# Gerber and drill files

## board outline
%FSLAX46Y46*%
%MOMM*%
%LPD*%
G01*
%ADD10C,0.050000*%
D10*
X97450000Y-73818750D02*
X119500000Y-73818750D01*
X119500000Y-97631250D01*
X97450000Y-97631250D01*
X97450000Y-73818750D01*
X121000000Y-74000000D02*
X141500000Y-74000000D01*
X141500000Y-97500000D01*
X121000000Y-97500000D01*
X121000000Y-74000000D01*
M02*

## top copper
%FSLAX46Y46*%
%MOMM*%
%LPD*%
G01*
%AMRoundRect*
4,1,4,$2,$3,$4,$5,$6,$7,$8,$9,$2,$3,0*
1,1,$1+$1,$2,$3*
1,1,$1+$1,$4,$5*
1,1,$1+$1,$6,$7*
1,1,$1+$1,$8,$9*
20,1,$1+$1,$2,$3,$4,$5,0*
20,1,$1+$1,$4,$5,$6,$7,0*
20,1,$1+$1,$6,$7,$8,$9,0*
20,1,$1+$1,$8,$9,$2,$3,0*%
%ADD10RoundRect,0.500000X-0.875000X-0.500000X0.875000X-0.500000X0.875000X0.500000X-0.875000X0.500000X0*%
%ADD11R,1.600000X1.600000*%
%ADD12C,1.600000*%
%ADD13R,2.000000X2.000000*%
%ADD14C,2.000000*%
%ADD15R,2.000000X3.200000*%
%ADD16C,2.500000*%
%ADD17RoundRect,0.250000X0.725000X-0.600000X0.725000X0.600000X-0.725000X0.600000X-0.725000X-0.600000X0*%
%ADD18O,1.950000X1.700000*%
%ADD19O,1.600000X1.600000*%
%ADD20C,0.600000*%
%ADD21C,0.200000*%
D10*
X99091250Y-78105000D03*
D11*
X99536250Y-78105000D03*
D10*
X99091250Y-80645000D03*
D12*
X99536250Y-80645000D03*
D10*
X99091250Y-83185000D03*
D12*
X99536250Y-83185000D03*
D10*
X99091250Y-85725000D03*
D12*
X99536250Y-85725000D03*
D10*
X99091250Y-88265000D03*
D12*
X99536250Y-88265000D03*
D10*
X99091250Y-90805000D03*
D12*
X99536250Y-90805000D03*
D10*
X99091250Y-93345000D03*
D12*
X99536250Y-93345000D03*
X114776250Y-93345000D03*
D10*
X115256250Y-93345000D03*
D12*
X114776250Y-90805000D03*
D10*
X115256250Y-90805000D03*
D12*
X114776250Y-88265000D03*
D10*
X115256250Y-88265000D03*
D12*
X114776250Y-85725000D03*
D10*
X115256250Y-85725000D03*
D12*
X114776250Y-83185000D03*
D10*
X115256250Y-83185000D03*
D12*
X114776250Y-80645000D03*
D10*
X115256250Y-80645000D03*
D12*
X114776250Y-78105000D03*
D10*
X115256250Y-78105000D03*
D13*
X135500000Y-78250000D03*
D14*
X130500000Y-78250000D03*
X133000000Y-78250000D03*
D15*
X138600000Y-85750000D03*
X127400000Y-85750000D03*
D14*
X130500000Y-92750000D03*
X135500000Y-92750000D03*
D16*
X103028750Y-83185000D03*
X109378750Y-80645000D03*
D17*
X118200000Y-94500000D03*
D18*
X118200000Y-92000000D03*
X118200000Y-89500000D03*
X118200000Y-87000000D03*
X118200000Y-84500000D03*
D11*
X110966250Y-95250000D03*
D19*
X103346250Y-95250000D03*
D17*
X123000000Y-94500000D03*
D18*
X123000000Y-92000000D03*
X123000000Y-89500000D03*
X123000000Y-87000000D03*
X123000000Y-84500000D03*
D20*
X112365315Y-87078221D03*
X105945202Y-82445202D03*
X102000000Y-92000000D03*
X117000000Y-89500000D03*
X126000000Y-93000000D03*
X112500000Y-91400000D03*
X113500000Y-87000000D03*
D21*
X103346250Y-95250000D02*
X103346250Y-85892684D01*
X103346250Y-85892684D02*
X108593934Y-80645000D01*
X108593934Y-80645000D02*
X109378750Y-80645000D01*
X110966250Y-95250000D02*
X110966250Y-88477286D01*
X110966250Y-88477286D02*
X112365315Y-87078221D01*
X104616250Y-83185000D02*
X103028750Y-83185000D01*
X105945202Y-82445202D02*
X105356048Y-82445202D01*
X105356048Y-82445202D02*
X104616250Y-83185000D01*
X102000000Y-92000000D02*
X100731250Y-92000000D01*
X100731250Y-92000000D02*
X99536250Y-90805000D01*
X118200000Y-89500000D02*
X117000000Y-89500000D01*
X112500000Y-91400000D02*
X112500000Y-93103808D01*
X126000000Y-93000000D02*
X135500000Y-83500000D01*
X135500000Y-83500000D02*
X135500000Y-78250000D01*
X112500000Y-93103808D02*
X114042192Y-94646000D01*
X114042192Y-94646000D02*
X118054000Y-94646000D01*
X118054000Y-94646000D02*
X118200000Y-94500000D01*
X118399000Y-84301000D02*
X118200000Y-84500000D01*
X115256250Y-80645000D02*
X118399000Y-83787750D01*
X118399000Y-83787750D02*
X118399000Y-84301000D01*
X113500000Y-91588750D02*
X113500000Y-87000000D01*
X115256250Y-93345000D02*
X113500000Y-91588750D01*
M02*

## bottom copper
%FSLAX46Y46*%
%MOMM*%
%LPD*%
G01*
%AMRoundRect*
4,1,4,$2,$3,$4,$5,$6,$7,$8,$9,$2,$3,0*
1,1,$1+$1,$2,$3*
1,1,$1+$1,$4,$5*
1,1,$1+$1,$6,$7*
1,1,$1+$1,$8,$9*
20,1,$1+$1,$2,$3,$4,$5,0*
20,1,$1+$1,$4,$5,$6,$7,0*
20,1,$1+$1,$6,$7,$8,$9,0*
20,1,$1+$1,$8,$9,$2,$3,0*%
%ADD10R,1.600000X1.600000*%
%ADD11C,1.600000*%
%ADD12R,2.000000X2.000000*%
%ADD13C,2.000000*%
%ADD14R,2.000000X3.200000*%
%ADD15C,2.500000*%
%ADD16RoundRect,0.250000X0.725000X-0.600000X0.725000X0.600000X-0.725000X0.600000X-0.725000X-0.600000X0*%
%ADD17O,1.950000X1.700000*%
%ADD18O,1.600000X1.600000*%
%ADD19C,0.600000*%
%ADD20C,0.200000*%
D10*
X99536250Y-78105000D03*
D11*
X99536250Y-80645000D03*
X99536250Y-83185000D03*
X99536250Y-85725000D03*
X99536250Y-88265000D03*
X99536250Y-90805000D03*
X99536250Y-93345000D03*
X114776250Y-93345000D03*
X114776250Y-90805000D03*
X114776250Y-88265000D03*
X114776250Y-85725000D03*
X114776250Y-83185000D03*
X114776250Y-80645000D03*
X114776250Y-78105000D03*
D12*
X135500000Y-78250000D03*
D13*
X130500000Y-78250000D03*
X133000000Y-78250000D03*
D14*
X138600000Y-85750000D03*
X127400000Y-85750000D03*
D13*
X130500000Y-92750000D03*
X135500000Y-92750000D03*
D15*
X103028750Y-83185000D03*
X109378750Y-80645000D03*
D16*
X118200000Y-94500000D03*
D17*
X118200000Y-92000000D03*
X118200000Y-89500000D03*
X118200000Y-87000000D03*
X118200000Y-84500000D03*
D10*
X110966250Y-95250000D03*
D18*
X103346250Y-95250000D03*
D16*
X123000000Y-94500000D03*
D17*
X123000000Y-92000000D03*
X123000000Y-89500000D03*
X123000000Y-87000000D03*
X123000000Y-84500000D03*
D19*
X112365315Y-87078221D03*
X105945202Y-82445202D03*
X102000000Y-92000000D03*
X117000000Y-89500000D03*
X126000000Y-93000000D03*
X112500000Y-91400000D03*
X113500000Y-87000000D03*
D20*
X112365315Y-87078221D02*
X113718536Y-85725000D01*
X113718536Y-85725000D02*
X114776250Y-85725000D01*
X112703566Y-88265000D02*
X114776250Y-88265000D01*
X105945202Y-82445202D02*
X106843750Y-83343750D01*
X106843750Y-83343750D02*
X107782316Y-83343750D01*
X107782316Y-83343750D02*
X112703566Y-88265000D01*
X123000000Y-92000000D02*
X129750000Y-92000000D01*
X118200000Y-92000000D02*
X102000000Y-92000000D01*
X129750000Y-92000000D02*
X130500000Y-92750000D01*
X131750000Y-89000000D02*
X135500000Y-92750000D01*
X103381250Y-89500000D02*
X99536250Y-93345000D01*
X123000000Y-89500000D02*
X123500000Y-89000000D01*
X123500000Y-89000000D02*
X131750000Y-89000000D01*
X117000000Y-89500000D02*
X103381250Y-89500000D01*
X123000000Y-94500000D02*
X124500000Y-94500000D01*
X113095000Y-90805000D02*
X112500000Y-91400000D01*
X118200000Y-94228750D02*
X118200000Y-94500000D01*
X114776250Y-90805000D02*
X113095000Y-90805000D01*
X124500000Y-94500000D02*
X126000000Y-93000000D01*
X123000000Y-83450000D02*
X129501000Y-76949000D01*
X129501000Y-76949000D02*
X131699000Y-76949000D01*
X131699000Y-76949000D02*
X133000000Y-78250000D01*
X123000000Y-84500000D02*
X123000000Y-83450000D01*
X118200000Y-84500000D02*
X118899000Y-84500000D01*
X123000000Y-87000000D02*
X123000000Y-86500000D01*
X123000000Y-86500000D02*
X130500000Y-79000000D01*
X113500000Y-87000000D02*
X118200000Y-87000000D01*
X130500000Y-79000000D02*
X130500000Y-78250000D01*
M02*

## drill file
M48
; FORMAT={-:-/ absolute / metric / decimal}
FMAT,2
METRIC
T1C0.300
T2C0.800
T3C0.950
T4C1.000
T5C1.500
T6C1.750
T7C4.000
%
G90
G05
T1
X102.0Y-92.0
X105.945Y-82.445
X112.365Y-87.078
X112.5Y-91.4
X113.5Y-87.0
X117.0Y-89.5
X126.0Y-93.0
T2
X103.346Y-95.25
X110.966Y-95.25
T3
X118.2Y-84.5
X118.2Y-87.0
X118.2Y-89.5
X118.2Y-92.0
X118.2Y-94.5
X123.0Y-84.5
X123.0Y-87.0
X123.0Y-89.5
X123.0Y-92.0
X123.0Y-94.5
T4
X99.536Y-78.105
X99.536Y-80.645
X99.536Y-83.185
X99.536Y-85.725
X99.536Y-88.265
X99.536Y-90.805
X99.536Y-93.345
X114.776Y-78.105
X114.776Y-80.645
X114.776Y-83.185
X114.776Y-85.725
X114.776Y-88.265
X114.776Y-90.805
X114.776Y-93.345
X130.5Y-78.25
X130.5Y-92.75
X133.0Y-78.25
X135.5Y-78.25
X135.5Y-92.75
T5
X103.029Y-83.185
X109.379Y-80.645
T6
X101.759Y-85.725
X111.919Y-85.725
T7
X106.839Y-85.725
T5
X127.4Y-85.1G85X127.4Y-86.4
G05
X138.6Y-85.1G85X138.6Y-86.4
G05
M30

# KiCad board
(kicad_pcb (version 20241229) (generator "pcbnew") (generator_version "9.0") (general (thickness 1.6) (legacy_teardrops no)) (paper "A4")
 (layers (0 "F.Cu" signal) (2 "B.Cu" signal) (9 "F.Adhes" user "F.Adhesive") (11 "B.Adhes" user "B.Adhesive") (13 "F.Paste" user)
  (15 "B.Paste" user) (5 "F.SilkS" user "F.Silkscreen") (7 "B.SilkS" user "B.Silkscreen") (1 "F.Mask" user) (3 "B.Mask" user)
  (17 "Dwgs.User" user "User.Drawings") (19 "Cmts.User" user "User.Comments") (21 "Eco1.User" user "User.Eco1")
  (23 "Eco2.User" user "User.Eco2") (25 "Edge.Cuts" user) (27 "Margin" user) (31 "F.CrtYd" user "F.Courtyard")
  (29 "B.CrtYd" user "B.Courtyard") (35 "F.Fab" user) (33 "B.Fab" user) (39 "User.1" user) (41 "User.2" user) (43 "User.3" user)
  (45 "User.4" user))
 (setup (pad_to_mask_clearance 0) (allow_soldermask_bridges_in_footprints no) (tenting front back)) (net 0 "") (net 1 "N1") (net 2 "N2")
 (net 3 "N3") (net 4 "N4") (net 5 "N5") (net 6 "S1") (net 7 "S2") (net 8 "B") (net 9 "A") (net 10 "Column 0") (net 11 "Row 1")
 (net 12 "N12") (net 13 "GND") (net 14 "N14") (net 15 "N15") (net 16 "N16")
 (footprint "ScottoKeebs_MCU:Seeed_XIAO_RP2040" (layer "F.Cu") (at 107.15625 85.725)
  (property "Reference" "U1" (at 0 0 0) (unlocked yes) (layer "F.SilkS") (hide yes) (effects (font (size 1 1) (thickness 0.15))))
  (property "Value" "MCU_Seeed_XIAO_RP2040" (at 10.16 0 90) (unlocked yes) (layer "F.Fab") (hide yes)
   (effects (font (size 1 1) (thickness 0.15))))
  (pad "1" smd roundrect (at -8.065 -7.62) (size 2.75 2) (layers "F.Cu" "F.Mask" "F.Paste") (roundrect_rratio 0.25) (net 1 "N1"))
  (pad "1" thru_hole rect (at -7.62 -7.62 90) (size 1.6 1.6) (drill 1) (layers "*.Cu" "*.Mask") (remove_unused_layers no) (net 1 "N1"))
  (pad "2" smd roundrect (at -8.065 -5.08) (size 2.75 2) (layers "F.Cu" "F.Mask" "F.Paste") (roundrect_rratio 0.25) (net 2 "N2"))
  (pad "2" thru_hole circle (at -7.62 -5.08 90) (size 1.6 1.6) (drill 1) (layers "*.Cu" "*.Mask") (remove_unused_layers no) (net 2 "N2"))
  (pad "3" smd roundrect (at -8.065 -2.54) (size 2.75 2) (layers "F.Cu" "F.Mask" "F.Paste") (roundrect_rratio 0.25) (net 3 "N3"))
  (pad "3" thru_hole circle (at -7.62 -2.54 90) (size 1.6 1.6) (drill 1) (layers "*.Cu" "*.Mask") (remove_unused_layers no) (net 3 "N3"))
  (pad "4" smd roundrect (at -8.065 0) (size 2.75 2) (layers "F.Cu" "F.Mask" "F.Paste") (roundrect_rratio 0.25) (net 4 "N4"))
  (pad "4" thru_hole circle (at -7.62 0 90) (size 1.6 1.6) (drill 1) (layers "*.Cu" "*.Mask") (remove_unused_layers no) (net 4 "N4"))
  (pad "5" smd roundrect (at -8.065 2.54) (size 2.75 2) (layers "F.Cu" "F.Mask" "F.Paste") (roundrect_rratio 0.25) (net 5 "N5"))
  (pad "5" thru_hole circle (at -7.62 2.54 90) (size 1.6 1.6) (drill 1) (layers "*.Cu" "*.Mask") (remove_unused_layers no) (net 5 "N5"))
  (pad "6" smd roundrect (at -8.065 5.08) (size 2.75 2) (layers "F.Cu" "F.Mask" "F.Paste") (roundrect_rratio 0.25) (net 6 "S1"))
  (pad "6" thru_hole circle (at -7.62 5.08 90) (size 1.6 1.6) (drill 1) (layers "*.Cu" "*.Mask") (remove_unused_layers no) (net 6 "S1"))
  (pad "7" smd roundrect (at -8.065 7.62) (size 2.75 2) (layers "F.Cu" "F.Mask" "F.Paste") (roundrect_rratio 0.25) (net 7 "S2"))
  (pad "7" thru_hole circle (at -7.62 7.62 90) (size 1.6 1.6) (drill 1) (layers "*.Cu" "*.Mask") (remove_unused_layers no) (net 7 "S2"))
  (pad "8" thru_hole circle (at 7.62 7.62 90) (size 1.6 1.6) (drill 1) (layers "*.Cu" "*.Mask") (remove_unused_layers no) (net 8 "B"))
  (pad "8" smd roundrect (at 8.1 7.62) (size 2.75 2) (layers "F.Cu" "F.Mask" "F.Paste") (roundrect_rratio 0.25) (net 8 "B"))
  (pad "9" thru_hole circle (at 7.62 5.08 90) (size 1.6 1.6) (drill 1) (layers "*.Cu" "*.Mask") (remove_unused_layers no) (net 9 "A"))
  (pad "9" smd roundrect (at 8.1 5.08) (size 2.75 2) (layers "F.Cu" "F.Mask" "F.Paste") (roundrect_rratio 0.25) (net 9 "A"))
  (pad "10" thru_hole circle (at 7.62 2.54 90) (size 1.6 1.6) (drill 1) (layers "*.Cu" "*.Mask") (remove_unused_layers no)
   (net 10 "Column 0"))
  (pad "10" smd roundrect (at 8.1 2.54) (size 2.75 2) (layers "F.Cu" "F.Mask" "F.Paste") (roundrect_rratio 0.25) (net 10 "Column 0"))
  (pad "11" thru_hole circle (at 7.62 0 90) (size 1.6 1.6) (drill 1) (layers "*.Cu" "*.Mask") (remove_unused_layers no) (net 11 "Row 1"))
  (pad "11" smd roundrect (at 8.1 0) (size 2.75 2) (layers "F.Cu" "F.Mask" "F.Paste") (roundrect_rratio 0.25) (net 11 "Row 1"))
  (pad "12" thru_hole circle (at 7.62 -2.54 90) (size 1.6 1.6) (drill 1) (layers "*.Cu" "*.Mask") (remove_unused_layers no) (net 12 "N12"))
  (pad "12" smd roundrect (at 8.1 -2.54) (size 2.75 2) (layers "F.Cu" "F.Mask" "F.Paste") (roundrect_rratio 0.25) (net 12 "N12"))
  (pad "13" thru_hole circle (at 7.62 -5.08 90) (size 1.6 1.6) (drill 1) (layers "*.Cu" "*.Mask") (remove_unused_layers no) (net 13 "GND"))
  (pad "13" smd roundrect (at 8.1 -5.08) (size 2.75 2) (layers "F.Cu" "F.Mask" "F.Paste") (roundrect_rratio 0.25) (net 13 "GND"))
  (pad "14" thru_hole circle (at 7.62 -7.62 90) (size 1.6 1.6) (drill 1) (layers "*.Cu" "*.Mask") (remove_unused_layers no) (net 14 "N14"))
  (pad "14" smd roundrect (at 8.1 -7.62) (size 2.75 2) (layers "F.Cu" "F.Mask" "F.Paste") (roundrect_rratio 0.25) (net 14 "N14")))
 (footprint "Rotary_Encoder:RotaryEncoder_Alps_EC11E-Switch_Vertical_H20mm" (layer "F.Cu") (at 135.5 78.25 -90)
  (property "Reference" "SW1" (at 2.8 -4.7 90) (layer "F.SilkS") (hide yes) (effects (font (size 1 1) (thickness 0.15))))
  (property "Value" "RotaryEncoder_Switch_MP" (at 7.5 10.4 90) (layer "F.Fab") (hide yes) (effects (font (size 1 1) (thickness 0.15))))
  (pad "A" thru_hole rect (at 0 0 270) (size 2 2) (drill 1) (layers "*.Cu" "*.Mask") (remove_unused_layers no) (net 9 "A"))
  (pad "B" thru_hole circle (at 0 5 270) (size 2 2) (drill 1) (layers "*.Cu" "*.Mask") (remove_unused_layers no) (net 8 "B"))
  (pad "C" thru_hole circle (at 0 2.5 270) (size 2 2) (drill 1) (layers "*.Cu" "*.Mask") (remove_unused_layers no) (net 13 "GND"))
  (pad "MP" thru_hole rect (at 7.5 -3.1 270) (size 3.2 2) (drill oval 2.8 1.5) (layers "*.Cu" "*.Mask") (remove_unused_layers no)
   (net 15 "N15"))
  (pad "MP" thru_hole rect (at 7.5 8.1 270) (size 3.2 2) (drill oval 2.8 1.5) (layers "*.Cu" "*.Mask") (remove_unused_layers no)
   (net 15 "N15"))
  (pad "S1" thru_hole circle (at 14.5 5 270) (size 2 2) (drill 1) (layers "*.Cu" "*.Mask") (remove_unused_layers no) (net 6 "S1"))
  (pad "S2" thru_hole circle (at 14.5 0 270) (size 2 2) (drill 1) (layers "*.Cu" "*.Mask") (remove_unused_layers no) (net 7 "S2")))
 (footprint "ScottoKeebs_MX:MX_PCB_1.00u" (layer "F.Cu") (at 106.83875 85.725)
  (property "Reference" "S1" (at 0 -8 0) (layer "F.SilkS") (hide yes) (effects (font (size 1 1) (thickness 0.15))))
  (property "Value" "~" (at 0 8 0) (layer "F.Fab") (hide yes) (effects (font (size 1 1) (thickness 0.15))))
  (pad "" np_thru_hole circle (at -5.08 0) (size 1.75 1.75) (drill 1.75) (layers "*.Cu" "*.Mask"))
  (pad "" np_thru_hole circle (at 0 0) (size 4 4) (drill 4) (layers "*.Cu" "*.Mask"))
  (pad "" np_thru_hole circle (at 5.08 0) (size 1.75 1.75) (drill 1.75) (layers "*.Cu" "*.Mask"))
  (pad "1" thru_hole circle (at -3.81 -2.54) (size 2.5 2.5) (drill 1.5) (layers "*.Cu" "*.Mask") (remove_unused_layers no)
   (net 10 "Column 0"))
  (pad "2" thru_hole circle (at 2.54 -5.08) (size 2.5 2.5) (drill 1.5) (layers "*.Cu" "*.Mask") (remove_unused_layers no) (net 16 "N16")))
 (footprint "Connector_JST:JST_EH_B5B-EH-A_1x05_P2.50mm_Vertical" (layer "F.Cu") (at 118.2 94.5 90)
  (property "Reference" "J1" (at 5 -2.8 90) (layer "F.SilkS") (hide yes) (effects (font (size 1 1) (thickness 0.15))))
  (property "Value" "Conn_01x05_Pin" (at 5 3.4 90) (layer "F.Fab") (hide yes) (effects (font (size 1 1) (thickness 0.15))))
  (pad "1" thru_hole roundrect (at 0 0 90) (size 1.7 1.95) (drill 0.95) (layers "*.Cu" "*.Mask") (remove_unused_layers no)
   (roundrect_rratio 0.147059) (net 9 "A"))
  (pad "2" thru_hole oval (at 2.5 0 90) (size 1.7 1.95) (drill 0.95) (layers "*.Cu" "*.Mask") (remove_unused_layers no) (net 6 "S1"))
  (pad "3" thru_hole oval (at 5 0 90) (size 1.7 1.95) (drill 0.95) (layers "*.Cu" "*.Mask") (remove_unused_layers no) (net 7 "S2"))
  (pad "4" thru_hole oval (at 7.5 0 90) (size 1.7 1.95) (drill 0.95) (layers "*.Cu" "*.Mask") (remove_unused_layers no) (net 8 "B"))
  (pad "5" thru_hole oval (at 10 0 90) (size 1.7 1.95) (drill 0.95) (layers "*.Cu" "*.Mask") (remove_unused_layers no) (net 13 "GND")))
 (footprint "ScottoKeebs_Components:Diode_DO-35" (layer "F.Cu") (at 110.96625 95.25 180)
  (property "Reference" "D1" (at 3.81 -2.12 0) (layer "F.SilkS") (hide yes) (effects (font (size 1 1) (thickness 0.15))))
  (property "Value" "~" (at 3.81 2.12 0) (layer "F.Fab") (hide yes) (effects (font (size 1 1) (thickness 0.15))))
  (pad "1" thru_hole rect (at 0 0 180) (size 1.6 1.6) (drill 0.8) (layers "*.Cu" "*.Mask") (remove_unused_layers no) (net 11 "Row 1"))
  (pad "2" thru_hole oval (at 7.62 0 180) (size 1.6 1.6) (drill 0.8) (layers "*.Cu" "*.Mask") (remove_unused_layers no) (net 16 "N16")))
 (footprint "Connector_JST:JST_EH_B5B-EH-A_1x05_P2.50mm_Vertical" (layer "F.Cu") (at 123 94.5 90)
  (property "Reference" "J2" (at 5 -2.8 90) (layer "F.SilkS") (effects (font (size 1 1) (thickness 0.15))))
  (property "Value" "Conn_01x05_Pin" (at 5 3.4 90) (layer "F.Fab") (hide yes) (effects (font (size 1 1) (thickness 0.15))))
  (pad "1" thru_hole roundrect (at 0 0 90) (size 1.7 1.95) (drill 0.95) (layers "*.Cu" "*.Mask") (remove_unused_layers no)
   (roundrect_rratio 0.147059) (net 9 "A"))
  (pad "2" thru_hole oval (at 2.5 0 90) (size 1.7 1.95) (drill 0.95) (layers "*.Cu" "*.Mask") (remove_unused_layers no) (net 6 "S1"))
  (pad "3" thru_hole oval (at 5 0 90) (size 1.7 1.95) (drill 0.95) (layers "*.Cu" "*.Mask") (remove_unused_layers no) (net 7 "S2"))
  (pad "4" thru_hole oval (at 7.5 0 90) (size 1.7 1.95) (drill 0.95) (layers "*.Cu" "*.Mask") (remove_unused_layers no) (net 8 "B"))
  (pad "5" thru_hole oval (at 10 0 90) (size 1.7 1.95) (drill 0.95) (layers "*.Cu" "*.Mask") (remove_unused_layers no) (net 13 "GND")))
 (gr_rect (start 97.45 73.81875) (end 119.5 97.63125) (stroke (width 0.05) (type default)) (fill no) (layer "Edge.Cuts"))
 (gr_rect (start 121 74) (end 141.5 97.5) (stroke (width 0.05) (type default)) (fill no) (layer "Edge.Cuts"))
 (segment (start 103.34625 95.25) (end 103.34625 85.892684) (width 0.2) (layer "F.Cu") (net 16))
 (segment (start 103.34625 85.892684) (end 108.593934 80.645) (width 0.2) (layer "F.Cu") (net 16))
 (segment (start 108.593934 80.645) (end 109.37875 80.645) (width 0.2) (layer "F.Cu") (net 16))
 (segment (start 110.96625 95.25) (end 110.96625 88.477286) (width 0.2) (layer "F.Cu") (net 11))
 (segment (start 110.96625 88.477286) (end 112.365315 87.078221) (width 0.2) (layer "F.Cu") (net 11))
 (via (at 112.365315 87.078221) (size 0.6) (drill 0.3) (layers "F.Cu" "B.Cu") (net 11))
 (segment (start 112.365315 87.078221) (end 113.718536 85.725) (width 0.2) (layer "B.Cu") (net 11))
 (segment (start 113.718536 85.725) (end 114.77625 85.725) (width 0.2) (layer "B.Cu") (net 11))
 (segment (start 104.61625 83.185) (end 103.02875 83.185) (width 0.2) (layer "F.Cu") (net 10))
 (segment (start 105.945202 82.445202) (end 105.356048 82.445202) (width 0.2) (layer "F.Cu") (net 10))
 (segment (start 105.356048 82.445202) (end 104.61625 83.185) (width 0.2) (layer "F.Cu") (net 10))
 (via (at 105.945202 82.445202) (size 0.6) (drill 0.3) (layers "F.Cu" "B.Cu") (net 10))
 (segment (start 112.703566 88.265) (end 114.77625 88.265) (width 0.2) (layer "B.Cu") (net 10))
 (segment (start 105.945202 82.445202) (end 106.84375 83.34375) (width 0.2) (layer "B.Cu") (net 10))
 (segment (start 106.84375 83.34375) (end 107.782316 83.34375) (width 0.2) (layer "B.Cu") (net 10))
 (segment (start 107.782316 83.34375) (end 112.703566 88.265) (width 0.2) (layer "B.Cu") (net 10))
 (segment (start 102 92) (end 100.73125 92) (width 0.2) (layer "F.Cu") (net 6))
 (segment (start 100.73125 92) (end 99.53625 90.805) (width 0.2) (layer "F.Cu") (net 6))
 (via (at 102 92) (size 0.6) (drill 0.3) (layers "F.Cu" "B.Cu") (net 6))
 (segment (start 123 92) (end 129.75 92) (width 0.2) (layer "B.Cu") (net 6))
 (segment (start 118.2 92) (end 102 92) (width 0.2) (layer "B.Cu") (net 6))
 (segment (start 129.75 92) (end 130.5 92.75) (width 0.2) (layer "B.Cu") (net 6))
 (segment (start 118.2 89.5) (end 117 89.5) (width 0.2) (layer "F.Cu") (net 7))
 (via (at 117 89.5) (size 0.6) (drill 0.3) (layers "F.Cu" "B.Cu") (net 7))
 (segment (start 131.75 89) (end 135.5 92.75) (width 0.2) (layer "B.Cu") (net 7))
 (segment (start 103.38125 89.5) (end 99.53625 93.345) (width 0.2) (layer "B.Cu") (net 7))
 (segment (start 123 89.5) (end 123.5 89) (width 0.2) (layer "B.Cu") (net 7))
 (segment (start 123.5 89) (end 131.75 89) (width 0.2) (layer "B.Cu") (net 7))
 (segment (start 117 89.5) (end 103.38125 89.5) (width 0.2) (layer "B.Cu") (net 7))
 (segment (start 112.5 91.4) (end 112.5 93.103808) (width 0.2) (layer "F.Cu") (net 9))
 (segment (start 126 93) (end 135.5 83.5) (width 0.2) (layer "F.Cu") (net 9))
 (segment (start 135.5 83.5) (end 135.5 78.25) (width 0.2) (layer "F.Cu") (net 9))
 (segment (start 112.5 93.103808) (end 114.042192 94.646) (width 0.2) (layer "F.Cu") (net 9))
 (segment (start 114.042192 94.646) (end 118.054 94.646) (width 0.2) (layer "F.Cu") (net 9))
 (segment (start 118.054 94.646) (end 118.2 94.5) (width 0.2) (layer "F.Cu") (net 9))
 (via (at 126 93) (size 0.6) (drill 0.3) (layers "F.Cu" "B.Cu") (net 9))
 (via (at 112.5 91.4) (size 0.6) (drill 0.3) (layers "F.Cu" "B.Cu") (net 9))
 (segment (start 123 94.5) (end 124.5 94.5) (width 0.2) (layer "B.Cu") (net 9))
 (segment (start 113.095 90.805) (end 112.5 91.4) (width 0.2) (layer "B.Cu") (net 9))
 (segment (start 118.2 94.22875) (end 118.2 94.5) (width 0.2) (layer "B.Cu") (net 9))
 (segment (start 114.77625 90.805) (end 113.095 90.805) (width 0.2) (layer "B.Cu") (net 9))
 (segment (start 124.5 94.5) (end 126 93) (width 0.2) (layer "B.Cu") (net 9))
 (segment (start 118.399 84.301) (end 118.2 84.5) (width 0.2) (layer "F.Cu") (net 13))
 (segment (start 115.25625 80.645) (end 118.399 83.78775) (width 0.2) (layer "F.Cu") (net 13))
 (segment (start 118.399 83.78775) (end 118.399 84.301) (width 0.2) (layer "F.Cu") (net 13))
 (segment (start 123 83.45) (end 129.501 76.949) (width 0.2) (layer "B.Cu") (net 13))
 (segment (start 129.501 76.949) (end 131.699 76.949) (width 0.2) (layer "B.Cu") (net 13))
 (segment (start 131.699 76.949) (end 133 78.25) (width 0.2) (layer "B.Cu") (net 13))
 (segment (start 123 84.5) (end 123 83.45) (width 0.2) (layer "B.Cu") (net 13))
 (segment (start 118.2 84.5) (end 118.899 84.5) (width 0.2) (layer "B.Cu") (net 13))
 (segment (start 113.5 91.58875) (end 113.5 87) (width 0.2) (layer "F.Cu") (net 8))
 (segment (start 115.25625 93.345) (end 113.5 91.58875) (width 0.2) (layer "F.Cu") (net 8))
 (via (at 113.5 87) (size 0.6) (drill 0.3) (layers "F.Cu" "B.Cu") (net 8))
 (segment (start 123 87) (end 123 86.5) (width 0.2) (layer "B.Cu") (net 8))
 (segment (start 123 86.5) (end 130.5 79) (width 0.2) (layer "B.Cu") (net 8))
 (segment (start 113.5 87) (end 118.2 87) (width 0.2) (layer "B.Cu") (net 8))
 (segment (start 130.5 79) (end 130.5 78.25) (width 0.2) (layer "B.Cu") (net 8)))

